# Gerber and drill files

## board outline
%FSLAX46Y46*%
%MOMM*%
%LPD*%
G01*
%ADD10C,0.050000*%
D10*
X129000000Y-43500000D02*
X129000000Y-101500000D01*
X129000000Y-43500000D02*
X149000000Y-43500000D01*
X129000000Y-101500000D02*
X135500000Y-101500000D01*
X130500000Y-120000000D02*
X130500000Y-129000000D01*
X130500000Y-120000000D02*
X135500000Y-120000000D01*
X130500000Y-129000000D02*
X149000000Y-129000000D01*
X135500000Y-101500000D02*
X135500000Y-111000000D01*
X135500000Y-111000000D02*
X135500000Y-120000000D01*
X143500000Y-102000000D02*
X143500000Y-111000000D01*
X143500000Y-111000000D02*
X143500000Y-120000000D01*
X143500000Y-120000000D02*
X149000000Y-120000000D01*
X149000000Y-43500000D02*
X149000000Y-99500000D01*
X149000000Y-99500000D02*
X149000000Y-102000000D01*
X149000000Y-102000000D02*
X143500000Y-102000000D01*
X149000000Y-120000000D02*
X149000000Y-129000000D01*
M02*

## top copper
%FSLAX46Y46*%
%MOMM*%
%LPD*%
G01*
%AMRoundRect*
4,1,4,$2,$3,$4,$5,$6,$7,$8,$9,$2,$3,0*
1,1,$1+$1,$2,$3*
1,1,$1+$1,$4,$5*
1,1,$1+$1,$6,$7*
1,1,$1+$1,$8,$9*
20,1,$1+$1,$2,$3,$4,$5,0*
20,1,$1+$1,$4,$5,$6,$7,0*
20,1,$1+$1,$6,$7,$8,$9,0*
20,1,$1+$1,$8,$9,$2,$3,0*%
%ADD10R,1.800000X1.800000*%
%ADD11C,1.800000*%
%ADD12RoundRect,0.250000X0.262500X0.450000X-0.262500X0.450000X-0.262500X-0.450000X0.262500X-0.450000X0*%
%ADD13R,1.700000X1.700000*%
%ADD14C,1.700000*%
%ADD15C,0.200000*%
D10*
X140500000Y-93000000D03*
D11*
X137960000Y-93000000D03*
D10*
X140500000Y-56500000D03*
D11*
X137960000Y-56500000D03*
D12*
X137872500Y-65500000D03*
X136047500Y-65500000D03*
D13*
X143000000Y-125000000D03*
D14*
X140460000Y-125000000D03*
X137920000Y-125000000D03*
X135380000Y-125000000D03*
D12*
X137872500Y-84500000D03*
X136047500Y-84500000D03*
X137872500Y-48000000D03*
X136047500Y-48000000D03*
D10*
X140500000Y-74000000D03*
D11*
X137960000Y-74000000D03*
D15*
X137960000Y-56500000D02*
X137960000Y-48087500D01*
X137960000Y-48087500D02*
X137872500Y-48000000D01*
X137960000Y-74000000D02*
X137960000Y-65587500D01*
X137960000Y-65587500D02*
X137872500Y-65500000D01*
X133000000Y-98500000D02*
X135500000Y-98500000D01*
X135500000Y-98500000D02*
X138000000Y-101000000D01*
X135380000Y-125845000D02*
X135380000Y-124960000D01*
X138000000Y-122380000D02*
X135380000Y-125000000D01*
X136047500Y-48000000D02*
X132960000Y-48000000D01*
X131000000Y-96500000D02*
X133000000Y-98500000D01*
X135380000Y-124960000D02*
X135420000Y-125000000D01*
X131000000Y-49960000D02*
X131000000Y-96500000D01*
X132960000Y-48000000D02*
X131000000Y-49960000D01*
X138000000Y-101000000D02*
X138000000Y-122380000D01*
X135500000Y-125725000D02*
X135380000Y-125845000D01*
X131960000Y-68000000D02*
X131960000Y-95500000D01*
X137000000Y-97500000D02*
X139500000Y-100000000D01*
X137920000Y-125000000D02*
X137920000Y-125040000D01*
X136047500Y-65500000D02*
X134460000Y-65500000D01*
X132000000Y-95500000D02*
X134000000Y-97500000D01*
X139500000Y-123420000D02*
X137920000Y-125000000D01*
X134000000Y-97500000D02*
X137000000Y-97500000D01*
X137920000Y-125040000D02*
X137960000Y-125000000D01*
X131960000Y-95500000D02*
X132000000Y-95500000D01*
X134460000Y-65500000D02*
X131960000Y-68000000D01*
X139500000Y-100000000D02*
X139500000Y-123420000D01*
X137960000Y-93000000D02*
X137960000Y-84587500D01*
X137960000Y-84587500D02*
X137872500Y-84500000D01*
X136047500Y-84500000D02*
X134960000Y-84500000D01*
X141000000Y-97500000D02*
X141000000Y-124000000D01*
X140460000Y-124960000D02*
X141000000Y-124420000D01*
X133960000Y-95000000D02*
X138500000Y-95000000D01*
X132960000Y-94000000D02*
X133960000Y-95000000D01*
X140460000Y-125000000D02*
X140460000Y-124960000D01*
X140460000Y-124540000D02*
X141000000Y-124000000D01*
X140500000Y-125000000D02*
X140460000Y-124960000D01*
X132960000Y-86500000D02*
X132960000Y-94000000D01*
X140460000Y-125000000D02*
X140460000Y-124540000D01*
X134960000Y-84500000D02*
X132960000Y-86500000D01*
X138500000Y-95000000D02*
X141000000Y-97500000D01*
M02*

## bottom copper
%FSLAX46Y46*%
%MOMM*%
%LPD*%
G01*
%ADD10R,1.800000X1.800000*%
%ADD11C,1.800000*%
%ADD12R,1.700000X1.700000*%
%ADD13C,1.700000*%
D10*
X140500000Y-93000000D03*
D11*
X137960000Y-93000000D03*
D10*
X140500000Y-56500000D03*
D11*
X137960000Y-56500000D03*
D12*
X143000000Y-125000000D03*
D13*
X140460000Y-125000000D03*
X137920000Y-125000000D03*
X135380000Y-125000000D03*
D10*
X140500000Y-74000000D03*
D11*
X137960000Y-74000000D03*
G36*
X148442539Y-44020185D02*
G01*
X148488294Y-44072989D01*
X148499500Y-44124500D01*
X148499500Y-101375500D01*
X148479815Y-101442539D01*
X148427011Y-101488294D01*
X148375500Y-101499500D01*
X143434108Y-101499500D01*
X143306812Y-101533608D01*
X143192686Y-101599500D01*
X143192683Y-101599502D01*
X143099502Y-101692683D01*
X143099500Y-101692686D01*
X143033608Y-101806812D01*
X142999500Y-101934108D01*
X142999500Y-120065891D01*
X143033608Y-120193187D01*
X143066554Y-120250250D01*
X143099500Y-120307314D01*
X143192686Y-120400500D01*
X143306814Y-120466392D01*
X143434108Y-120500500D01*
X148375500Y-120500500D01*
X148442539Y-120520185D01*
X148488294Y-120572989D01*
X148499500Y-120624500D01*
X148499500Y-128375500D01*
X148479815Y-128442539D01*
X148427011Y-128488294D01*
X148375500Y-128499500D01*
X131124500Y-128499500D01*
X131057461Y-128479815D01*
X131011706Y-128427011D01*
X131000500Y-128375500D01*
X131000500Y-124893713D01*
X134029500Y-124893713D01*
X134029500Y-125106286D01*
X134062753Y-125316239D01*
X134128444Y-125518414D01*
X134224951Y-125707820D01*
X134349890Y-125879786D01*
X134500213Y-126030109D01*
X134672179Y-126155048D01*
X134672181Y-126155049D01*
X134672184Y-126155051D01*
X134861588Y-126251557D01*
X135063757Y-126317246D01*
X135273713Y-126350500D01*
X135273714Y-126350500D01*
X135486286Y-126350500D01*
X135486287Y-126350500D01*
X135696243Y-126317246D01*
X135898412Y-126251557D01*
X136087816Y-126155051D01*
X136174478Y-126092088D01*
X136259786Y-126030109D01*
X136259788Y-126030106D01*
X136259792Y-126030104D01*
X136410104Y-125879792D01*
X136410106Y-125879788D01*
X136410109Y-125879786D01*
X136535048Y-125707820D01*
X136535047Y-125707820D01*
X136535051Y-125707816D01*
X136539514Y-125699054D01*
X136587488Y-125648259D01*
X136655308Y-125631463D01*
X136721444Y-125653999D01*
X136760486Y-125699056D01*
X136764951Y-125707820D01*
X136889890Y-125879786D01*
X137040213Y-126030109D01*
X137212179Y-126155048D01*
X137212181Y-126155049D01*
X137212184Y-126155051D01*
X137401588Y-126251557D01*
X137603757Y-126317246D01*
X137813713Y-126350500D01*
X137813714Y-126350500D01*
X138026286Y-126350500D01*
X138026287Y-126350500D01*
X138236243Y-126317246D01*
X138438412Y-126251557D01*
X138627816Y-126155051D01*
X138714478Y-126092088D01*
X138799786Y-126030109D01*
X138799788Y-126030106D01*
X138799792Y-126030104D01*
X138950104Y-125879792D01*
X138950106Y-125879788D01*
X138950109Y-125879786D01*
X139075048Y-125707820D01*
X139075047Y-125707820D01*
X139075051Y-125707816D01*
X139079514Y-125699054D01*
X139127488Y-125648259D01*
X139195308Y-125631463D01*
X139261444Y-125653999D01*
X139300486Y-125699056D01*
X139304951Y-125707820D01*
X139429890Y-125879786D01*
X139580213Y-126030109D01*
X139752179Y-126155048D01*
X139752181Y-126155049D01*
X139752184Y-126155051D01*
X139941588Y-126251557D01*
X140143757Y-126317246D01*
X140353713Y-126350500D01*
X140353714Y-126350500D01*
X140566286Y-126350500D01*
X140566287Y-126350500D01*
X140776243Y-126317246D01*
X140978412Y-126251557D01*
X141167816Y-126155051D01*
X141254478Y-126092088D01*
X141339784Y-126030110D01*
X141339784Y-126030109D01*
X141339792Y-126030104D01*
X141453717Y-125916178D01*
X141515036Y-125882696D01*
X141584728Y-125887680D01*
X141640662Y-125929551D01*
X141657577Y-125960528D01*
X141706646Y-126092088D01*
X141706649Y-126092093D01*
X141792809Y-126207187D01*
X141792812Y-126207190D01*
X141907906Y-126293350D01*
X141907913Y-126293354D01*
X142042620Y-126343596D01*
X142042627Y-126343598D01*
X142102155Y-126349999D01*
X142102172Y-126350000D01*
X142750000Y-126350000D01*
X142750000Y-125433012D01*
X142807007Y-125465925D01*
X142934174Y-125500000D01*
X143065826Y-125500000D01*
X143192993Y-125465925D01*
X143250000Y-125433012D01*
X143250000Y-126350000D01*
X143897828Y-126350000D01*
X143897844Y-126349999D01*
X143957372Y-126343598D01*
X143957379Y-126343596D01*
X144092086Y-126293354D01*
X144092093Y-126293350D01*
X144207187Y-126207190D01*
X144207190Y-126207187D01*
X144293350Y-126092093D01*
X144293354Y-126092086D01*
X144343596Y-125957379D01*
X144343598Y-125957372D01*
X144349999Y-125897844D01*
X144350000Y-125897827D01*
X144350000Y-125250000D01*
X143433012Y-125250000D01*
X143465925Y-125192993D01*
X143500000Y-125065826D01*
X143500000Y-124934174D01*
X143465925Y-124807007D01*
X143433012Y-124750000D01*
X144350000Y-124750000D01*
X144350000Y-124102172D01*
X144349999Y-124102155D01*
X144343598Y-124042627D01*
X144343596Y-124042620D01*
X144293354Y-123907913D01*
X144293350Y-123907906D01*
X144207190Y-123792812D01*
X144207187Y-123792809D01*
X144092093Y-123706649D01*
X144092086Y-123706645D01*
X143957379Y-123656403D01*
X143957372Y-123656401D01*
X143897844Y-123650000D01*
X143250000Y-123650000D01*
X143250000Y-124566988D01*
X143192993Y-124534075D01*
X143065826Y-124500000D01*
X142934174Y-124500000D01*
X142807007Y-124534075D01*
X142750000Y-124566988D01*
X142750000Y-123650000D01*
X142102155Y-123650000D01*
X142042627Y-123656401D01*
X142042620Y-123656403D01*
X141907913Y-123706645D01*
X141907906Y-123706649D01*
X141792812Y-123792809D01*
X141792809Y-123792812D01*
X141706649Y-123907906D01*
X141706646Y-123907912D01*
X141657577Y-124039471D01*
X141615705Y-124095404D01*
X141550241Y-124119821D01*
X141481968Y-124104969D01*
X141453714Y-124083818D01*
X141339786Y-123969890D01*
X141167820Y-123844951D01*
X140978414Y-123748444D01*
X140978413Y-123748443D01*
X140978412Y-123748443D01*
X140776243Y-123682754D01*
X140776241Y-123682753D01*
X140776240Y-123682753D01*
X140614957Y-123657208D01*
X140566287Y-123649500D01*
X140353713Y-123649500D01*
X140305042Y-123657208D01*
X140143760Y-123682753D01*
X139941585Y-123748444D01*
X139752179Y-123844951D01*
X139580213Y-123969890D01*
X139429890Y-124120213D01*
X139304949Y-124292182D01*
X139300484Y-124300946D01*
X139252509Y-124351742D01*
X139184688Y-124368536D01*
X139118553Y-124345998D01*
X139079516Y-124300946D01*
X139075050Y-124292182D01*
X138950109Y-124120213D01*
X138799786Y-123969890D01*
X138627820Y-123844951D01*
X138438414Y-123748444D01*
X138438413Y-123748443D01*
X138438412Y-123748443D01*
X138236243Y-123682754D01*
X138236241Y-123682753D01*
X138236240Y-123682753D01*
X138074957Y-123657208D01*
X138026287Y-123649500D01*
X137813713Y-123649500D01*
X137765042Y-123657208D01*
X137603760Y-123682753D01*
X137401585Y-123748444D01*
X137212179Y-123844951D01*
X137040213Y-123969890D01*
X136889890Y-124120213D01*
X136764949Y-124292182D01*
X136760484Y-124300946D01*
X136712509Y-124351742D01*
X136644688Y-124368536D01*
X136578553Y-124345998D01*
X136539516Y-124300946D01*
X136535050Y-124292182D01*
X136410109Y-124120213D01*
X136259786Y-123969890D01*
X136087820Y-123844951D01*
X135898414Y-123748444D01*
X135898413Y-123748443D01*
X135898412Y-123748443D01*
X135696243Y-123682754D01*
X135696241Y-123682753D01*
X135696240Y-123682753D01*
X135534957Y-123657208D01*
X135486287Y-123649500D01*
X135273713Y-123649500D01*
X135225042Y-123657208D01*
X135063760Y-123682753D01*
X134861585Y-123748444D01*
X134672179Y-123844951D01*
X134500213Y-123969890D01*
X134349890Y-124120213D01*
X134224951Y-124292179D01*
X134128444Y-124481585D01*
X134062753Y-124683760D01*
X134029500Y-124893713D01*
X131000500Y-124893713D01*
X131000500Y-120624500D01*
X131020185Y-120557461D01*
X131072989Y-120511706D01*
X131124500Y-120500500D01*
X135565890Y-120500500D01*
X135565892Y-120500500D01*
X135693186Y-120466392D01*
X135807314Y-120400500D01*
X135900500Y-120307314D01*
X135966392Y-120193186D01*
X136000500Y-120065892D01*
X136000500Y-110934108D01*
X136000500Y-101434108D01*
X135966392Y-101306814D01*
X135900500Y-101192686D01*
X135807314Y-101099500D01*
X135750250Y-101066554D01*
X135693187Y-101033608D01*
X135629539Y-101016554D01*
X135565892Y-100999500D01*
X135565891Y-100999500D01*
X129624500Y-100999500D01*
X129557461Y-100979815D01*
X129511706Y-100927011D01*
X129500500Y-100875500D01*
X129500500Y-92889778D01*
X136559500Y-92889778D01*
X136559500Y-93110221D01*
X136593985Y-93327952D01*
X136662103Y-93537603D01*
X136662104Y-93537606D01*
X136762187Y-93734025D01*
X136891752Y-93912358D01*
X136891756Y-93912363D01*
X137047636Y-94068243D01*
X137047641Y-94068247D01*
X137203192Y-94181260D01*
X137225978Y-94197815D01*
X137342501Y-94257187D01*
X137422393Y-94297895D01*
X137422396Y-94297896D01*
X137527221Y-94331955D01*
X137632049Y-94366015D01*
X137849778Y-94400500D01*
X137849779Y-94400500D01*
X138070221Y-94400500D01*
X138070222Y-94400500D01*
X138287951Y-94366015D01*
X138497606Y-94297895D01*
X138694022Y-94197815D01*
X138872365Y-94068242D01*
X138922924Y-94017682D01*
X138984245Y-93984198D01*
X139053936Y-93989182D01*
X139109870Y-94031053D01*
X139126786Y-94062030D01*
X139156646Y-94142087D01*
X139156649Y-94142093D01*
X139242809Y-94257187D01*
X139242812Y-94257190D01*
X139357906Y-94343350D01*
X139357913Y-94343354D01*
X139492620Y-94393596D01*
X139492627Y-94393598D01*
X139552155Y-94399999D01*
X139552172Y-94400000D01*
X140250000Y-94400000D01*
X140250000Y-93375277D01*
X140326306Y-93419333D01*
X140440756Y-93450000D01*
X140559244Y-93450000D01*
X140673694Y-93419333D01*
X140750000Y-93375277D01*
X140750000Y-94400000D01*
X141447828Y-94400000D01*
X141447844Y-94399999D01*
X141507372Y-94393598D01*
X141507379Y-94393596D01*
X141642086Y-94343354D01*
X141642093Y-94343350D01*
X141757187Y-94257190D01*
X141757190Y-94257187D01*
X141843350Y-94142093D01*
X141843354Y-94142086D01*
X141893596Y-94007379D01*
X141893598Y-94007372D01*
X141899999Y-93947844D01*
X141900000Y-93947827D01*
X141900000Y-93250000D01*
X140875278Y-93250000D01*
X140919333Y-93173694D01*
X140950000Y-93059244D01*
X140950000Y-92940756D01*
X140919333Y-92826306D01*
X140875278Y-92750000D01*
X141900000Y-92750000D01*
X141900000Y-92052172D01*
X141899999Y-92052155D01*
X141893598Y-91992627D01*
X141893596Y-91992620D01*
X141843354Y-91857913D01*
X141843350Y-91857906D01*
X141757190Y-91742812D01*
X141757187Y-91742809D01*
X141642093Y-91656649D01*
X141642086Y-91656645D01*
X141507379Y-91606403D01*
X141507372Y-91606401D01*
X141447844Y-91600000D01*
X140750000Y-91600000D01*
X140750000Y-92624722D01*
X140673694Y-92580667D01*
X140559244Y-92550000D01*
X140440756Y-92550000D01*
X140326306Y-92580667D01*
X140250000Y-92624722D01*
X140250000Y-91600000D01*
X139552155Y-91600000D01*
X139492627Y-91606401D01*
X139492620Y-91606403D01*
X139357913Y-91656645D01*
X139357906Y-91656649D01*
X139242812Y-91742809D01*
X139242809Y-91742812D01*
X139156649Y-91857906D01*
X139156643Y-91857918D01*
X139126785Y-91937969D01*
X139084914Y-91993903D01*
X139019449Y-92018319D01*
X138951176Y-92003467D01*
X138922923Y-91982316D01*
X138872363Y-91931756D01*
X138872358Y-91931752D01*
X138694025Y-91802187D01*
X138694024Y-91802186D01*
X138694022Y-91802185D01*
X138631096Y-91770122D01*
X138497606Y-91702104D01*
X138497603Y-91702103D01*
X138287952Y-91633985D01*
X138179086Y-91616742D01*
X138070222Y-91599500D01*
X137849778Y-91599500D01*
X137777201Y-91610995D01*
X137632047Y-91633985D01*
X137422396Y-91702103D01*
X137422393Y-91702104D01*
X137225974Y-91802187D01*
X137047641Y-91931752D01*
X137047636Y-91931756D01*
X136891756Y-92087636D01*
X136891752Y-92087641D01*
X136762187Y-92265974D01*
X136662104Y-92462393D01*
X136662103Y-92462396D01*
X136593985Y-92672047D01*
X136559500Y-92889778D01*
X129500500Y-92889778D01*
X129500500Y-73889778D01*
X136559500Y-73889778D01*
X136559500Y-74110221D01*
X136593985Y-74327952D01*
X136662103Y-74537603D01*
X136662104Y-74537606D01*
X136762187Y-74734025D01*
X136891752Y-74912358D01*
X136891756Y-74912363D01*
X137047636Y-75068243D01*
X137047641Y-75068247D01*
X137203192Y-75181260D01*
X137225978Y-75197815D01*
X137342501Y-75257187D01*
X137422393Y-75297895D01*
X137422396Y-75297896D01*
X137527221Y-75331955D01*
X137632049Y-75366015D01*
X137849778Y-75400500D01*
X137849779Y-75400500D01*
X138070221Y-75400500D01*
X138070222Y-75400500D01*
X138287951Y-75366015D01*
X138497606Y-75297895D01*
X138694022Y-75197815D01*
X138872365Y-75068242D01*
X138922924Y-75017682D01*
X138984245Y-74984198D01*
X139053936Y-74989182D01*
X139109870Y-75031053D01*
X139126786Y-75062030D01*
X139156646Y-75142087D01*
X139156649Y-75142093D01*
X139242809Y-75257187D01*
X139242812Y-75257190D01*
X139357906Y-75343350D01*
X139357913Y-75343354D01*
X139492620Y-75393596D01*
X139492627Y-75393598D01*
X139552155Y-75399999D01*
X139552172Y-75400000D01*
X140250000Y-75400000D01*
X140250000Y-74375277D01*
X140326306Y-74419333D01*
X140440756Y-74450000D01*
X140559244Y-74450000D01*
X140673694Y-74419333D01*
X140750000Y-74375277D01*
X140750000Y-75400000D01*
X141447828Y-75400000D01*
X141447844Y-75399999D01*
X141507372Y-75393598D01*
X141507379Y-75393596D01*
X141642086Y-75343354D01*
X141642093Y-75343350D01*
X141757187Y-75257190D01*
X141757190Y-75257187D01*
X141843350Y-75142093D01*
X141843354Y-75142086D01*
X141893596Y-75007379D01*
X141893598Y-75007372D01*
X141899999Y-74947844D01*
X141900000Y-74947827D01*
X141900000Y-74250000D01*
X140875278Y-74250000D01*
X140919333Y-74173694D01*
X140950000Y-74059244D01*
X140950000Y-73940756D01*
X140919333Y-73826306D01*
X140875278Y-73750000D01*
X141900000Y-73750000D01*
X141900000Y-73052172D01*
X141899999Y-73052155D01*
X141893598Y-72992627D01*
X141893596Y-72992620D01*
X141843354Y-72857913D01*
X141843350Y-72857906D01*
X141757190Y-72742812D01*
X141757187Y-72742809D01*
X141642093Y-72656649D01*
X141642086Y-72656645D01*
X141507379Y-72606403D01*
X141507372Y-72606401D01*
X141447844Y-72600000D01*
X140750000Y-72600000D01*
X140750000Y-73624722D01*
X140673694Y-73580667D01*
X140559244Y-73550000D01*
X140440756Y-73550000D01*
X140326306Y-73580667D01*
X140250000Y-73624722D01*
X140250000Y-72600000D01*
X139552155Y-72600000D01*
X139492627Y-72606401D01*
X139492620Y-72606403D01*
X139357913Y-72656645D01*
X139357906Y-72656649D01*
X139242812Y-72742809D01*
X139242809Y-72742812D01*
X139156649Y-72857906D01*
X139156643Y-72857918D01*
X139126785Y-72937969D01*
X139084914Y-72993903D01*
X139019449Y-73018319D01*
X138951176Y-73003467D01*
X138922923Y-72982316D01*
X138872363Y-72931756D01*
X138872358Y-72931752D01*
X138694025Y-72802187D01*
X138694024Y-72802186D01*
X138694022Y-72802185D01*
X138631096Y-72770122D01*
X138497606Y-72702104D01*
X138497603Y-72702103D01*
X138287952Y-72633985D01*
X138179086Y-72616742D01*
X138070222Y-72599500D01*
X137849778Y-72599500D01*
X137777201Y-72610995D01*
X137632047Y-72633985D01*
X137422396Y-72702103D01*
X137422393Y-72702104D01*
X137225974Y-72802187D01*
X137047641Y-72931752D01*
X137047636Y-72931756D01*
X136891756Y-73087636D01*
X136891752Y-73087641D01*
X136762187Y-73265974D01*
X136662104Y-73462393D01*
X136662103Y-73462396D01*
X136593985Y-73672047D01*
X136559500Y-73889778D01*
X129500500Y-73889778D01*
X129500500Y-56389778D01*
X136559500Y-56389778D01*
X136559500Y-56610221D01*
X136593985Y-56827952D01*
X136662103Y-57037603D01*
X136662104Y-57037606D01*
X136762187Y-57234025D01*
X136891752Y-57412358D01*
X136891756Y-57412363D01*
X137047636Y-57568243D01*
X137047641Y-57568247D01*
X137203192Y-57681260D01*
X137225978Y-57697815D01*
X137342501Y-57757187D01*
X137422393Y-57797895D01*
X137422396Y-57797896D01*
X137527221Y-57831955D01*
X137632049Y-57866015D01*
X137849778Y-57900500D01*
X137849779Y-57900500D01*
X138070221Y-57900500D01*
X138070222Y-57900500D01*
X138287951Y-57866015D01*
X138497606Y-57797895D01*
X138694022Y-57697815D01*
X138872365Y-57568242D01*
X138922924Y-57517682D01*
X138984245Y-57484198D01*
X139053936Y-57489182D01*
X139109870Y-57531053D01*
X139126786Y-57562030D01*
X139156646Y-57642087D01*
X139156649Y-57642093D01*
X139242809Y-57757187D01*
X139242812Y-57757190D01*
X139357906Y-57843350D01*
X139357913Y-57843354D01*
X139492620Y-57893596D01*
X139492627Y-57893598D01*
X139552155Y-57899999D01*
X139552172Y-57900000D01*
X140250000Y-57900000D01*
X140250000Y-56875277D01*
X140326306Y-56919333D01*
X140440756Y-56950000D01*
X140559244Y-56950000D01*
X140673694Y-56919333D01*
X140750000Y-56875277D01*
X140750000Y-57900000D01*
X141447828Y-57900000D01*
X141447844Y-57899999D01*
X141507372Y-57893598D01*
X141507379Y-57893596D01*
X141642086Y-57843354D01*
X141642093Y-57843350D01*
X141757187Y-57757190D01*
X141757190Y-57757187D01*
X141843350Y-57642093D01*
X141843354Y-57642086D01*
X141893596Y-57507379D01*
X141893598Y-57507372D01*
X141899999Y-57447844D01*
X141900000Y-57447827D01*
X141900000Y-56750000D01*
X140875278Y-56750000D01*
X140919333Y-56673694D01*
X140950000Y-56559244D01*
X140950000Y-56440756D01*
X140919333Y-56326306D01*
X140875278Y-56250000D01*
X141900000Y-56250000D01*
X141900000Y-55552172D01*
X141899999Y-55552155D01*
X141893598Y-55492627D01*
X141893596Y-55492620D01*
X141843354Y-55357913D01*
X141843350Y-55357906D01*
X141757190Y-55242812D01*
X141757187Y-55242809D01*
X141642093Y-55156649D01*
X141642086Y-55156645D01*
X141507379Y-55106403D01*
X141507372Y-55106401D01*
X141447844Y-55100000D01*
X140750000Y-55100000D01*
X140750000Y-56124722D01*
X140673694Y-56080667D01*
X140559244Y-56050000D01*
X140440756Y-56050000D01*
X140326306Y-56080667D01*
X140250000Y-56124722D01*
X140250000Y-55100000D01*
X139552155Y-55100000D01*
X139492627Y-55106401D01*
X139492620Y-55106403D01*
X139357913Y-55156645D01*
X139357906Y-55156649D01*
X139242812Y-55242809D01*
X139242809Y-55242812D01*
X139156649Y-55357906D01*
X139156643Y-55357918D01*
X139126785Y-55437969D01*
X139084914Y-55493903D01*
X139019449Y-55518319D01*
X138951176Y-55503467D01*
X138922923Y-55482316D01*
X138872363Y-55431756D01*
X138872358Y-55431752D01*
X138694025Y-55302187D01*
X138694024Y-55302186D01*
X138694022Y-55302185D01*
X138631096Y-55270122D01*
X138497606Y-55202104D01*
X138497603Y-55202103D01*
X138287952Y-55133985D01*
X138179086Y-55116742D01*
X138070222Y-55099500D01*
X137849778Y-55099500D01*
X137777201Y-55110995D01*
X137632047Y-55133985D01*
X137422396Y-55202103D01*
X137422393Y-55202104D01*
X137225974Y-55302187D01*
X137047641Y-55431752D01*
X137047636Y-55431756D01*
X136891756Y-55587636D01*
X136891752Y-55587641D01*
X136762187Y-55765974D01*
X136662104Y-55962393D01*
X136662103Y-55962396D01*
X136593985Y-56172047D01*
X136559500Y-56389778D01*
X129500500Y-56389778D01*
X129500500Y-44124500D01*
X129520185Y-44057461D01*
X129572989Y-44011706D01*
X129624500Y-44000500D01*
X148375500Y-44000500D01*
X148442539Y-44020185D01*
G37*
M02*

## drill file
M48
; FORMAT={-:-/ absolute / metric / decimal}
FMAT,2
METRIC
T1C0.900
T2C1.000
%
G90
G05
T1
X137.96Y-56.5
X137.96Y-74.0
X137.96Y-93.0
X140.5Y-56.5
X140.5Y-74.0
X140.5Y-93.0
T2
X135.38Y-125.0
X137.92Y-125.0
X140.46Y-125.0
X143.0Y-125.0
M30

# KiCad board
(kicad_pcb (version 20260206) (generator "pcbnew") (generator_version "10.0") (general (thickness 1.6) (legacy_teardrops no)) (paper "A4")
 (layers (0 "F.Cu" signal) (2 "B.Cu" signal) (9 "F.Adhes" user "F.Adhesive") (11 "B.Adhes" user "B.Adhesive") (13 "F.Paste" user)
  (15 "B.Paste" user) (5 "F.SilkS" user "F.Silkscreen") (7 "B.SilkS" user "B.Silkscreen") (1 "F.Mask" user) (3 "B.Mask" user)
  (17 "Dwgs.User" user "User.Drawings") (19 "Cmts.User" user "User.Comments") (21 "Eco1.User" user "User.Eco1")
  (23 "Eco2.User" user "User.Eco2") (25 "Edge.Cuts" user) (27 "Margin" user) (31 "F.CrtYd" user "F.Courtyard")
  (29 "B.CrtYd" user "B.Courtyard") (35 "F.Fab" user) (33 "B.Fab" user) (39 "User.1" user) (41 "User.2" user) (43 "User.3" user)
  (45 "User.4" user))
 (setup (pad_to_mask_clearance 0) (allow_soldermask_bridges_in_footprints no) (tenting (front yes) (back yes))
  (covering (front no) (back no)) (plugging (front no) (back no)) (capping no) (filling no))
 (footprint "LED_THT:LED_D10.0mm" (layer "F.Cu") (at 140.5 93 180)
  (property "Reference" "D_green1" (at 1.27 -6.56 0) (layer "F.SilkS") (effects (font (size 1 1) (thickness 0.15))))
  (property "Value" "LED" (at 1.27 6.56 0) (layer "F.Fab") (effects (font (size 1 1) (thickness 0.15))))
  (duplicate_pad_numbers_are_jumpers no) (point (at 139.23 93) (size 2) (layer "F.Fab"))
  (pad "1" thru_hole rect (at 0 0 180) (size 1.8 1.8) (drill 0.9) (layers "*.Cu" "*.Mask") (remove_unused_layers no) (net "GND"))
  (pad "2" thru_hole circle (at 2.54 0 180) (size 1.8 1.8) (drill 0.9) (layers "*.Cu" "*.Mask") (remove_unused_layers no)
   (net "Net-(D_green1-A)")))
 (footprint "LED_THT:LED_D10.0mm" (layer "F.Cu") (at 140.5 56.5 180)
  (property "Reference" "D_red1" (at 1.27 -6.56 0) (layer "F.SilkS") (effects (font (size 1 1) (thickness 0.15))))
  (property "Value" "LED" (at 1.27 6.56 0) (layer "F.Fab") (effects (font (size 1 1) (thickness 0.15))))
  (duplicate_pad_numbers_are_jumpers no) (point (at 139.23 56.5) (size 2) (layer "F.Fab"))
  (pad "1" thru_hole rect (at 0 0 180) (size 1.8 1.8) (drill 0.9) (layers "*.Cu" "*.Mask") (remove_unused_layers no) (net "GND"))
  (pad "2" thru_hole circle (at 2.54 0 180) (size 1.8 1.8) (drill 0.9) (layers "*.Cu" "*.Mask") (remove_unused_layers no)
   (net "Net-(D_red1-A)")))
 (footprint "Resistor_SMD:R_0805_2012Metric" (layer "F.Cu") (at 136.96 65.5 180)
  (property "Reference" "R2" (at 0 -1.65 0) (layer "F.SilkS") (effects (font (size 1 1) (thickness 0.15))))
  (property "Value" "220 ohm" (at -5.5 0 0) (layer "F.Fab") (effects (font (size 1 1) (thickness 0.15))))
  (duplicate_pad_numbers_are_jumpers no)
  (pad "1" smd roundrect (at -0.9125 0 180) (size 1.025 1.4) (layers "F.Cu" "F.Mask" "F.Paste") (roundrect_rratio 0.243902)
   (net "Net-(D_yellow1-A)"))
  (pad "2" smd roundrect (at 0.9125 0 180) (size 1.025 1.4) (layers "F.Cu" "F.Mask" "F.Paste") (roundrect_rratio 0.243902)
   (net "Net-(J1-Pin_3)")))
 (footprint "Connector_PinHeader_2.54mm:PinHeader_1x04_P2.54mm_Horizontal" (layer "F.Cu") (at 143 125 -90)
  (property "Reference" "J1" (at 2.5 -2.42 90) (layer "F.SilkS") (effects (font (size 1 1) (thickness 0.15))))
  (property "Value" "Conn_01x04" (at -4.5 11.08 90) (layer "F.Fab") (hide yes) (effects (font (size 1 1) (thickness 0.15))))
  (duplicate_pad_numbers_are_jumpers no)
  (pad "1" thru_hole rect (at 0 0 270) (size 1.7 1.7) (drill 1) (layers "*.Cu" "*.Mask") (remove_unused_layers no) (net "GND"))
  (pad "2" thru_hole circle (at 0 2.54 270) (size 1.7 1.7) (drill 1) (layers "*.Cu" "*.Mask") (remove_unused_layers no)
   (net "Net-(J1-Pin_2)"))
  (pad "3" thru_hole circle (at 0 5.08 270) (size 1.7 1.7) (drill 1) (layers "*.Cu" "*.Mask") (remove_unused_layers no)
   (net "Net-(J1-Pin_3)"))
  (pad "4" thru_hole circle (at 0 7.62 270) (size 1.7 1.7) (drill 1) (layers "*.Cu" "*.Mask") (remove_unused_layers no)
   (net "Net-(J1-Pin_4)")))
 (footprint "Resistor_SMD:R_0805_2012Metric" (layer "F.Cu") (at 136.96 84.5 180)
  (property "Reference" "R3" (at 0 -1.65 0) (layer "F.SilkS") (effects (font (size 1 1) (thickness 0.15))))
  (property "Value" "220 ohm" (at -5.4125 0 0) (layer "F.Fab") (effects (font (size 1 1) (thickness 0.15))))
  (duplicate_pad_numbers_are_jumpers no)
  (pad "1" smd roundrect (at -0.9125 0 180) (size 1.025 1.4) (layers "F.Cu" "F.Mask" "F.Paste") (roundrect_rratio 0.243902)
   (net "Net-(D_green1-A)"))
  (pad "2" smd roundrect (at 0.9125 0 180) (size 1.025 1.4) (layers "F.Cu" "F.Mask" "F.Paste") (roundrect_rratio 0.243902)
   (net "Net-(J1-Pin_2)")))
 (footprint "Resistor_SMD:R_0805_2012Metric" (layer "F.Cu") (at 136.96 48 180)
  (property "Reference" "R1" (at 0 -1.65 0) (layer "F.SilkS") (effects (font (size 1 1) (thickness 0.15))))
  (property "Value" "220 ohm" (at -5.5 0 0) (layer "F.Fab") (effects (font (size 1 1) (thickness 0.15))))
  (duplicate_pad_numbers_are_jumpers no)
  (pad "1" smd roundrect (at -0.9125 0 180) (size 1.025 1.4) (layers "F.Cu" "F.Mask" "F.Paste") (roundrect_rratio 0.243902)
   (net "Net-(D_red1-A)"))
  (pad "2" smd roundrect (at 0.9125 0 180) (size 1.025 1.4) (layers "F.Cu" "F.Mask" "F.Paste") (roundrect_rratio 0.243902)
   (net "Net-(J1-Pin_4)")))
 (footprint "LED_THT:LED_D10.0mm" (layer "F.Cu") (at 140.5 74 180)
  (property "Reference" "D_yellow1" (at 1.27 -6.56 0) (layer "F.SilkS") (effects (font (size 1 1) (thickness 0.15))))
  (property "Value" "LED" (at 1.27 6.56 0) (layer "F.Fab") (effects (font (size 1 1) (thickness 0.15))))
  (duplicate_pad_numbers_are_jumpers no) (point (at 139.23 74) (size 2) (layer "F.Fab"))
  (pad "1" thru_hole rect (at 0 0 180) (size 1.8 1.8) (drill 0.9) (layers "*.Cu" "*.Mask") (remove_unused_layers no) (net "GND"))
  (pad "2" thru_hole circle (at 2.54 0 180) (size 1.8 1.8) (drill 0.9) (layers "*.Cu" "*.Mask") (remove_unused_layers no)
   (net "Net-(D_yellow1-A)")))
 (gr_line (start 129 43.5) (end 129 101.5) (stroke (width 0.05) (type default)) (layer "Edge.Cuts"))
 (gr_line (start 129 43.5) (end 149 43.5) (stroke (width 0.05) (type default)) (layer "Edge.Cuts"))
 (gr_line (start 129 101.5) (end 135.5 101.5) (stroke (width 0.05) (type default)) (layer "Edge.Cuts"))
 (gr_line (start 130.5 120) (end 130.5 129) (stroke (width 0.05) (type default)) (layer "Edge.Cuts"))
 (gr_line (start 130.5 120) (end 135.5 120) (stroke (width 0.05) (type default)) (layer "Edge.Cuts"))
 (gr_line (start 130.5 129) (end 149 129) (stroke (width 0.05) (type default)) (layer "Edge.Cuts"))
 (gr_line (start 135.5 101.5) (end 135.5 111) (stroke (width 0.05) (type default)) (layer "Edge.Cuts"))
 (gr_line (start 135.5 111) (end 135.5 120) (stroke (width 0.05) (type default)) (layer "Edge.Cuts"))
 (gr_line (start 143.5 102) (end 143.5 111) (stroke (width 0.05) (type default)) (layer "Edge.Cuts"))
 (gr_line (start 143.5 111) (end 143.5 120) (stroke (width 0.05) (type default)) (layer "Edge.Cuts"))
 (gr_line (start 143.5 120) (end 149 120) (stroke (width 0.05) (type default)) (layer "Edge.Cuts"))
 (gr_line (start 149 43.5) (end 149 99.5) (stroke (width 0.05) (type default)) (layer "Edge.Cuts"))
 (gr_line (start 149 99.5) (end 149 102) (stroke (width 0.05) (type default)) (layer "Edge.Cuts"))
 (gr_line (start 149 102) (end 143.5 102) (stroke (width 0.05) (type default)) (layer "Edge.Cuts"))
 (gr_line (start 149 120) (end 149 129) (stroke (width 0.05) (type default)) (layer "Edge.Cuts"))
 (segment (start 137.96 56.5) (end 137.96 48.0875) (width 0.2) (layer "F.Cu") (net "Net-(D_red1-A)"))
 (segment (start 137.96 48.0875) (end 137.8725 48) (width 0.2) (layer "F.Cu") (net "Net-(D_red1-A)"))
 (segment (start 137.96 74) (end 137.96 65.5875) (width 0.2) (layer "F.Cu") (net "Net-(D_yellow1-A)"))
 (segment (start 137.96 65.5875) (end 137.8725 65.5) (width 0.2) (layer "F.Cu") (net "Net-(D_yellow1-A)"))
 (segment (start 133 98.5) (end 135.5 98.5) (width 0.2) (layer "F.Cu") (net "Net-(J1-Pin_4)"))
 (segment (start 135.5 98.5) (end 138 101) (width 0.2) (layer "F.Cu") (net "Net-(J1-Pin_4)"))
 (segment (start 135.38 125.845) (end 135.38 124.96) (width 0.2) (layer "F.Cu") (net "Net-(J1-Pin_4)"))
 (segment (start 138 122.38) (end 135.38 125) (width 0.2) (layer "F.Cu") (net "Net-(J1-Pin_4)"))
 (segment (start 136.0475 48) (end 132.96 48) (width 0.2) (layer "F.Cu") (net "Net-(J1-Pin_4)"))
 (segment (start 131 96.5) (end 133 98.5) (width 0.2) (layer "F.Cu") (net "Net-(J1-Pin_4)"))
 (segment (start 135.38 124.96) (end 135.42 125) (width 0.2) (layer "F.Cu") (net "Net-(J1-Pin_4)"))
 (segment (start 131 49.96) (end 131 96.5) (width 0.2) (layer "F.Cu") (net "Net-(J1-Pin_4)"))
 (segment (start 132.96 48) (end 131 49.96) (width 0.2) (layer "F.Cu") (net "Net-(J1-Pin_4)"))
 (segment (start 138 101) (end 138 122.38) (width 0.2) (layer "F.Cu") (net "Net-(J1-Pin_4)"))
 (segment (start 135.5 125.725) (end 135.38 125.845) (width 0.2) (layer "F.Cu") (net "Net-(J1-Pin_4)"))
 (segment (start 131.96 68) (end 131.96 95.5) (width 0.2) (layer "F.Cu") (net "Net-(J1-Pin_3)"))
 (segment (start 137 97.5) (end 139.5 100) (width 0.2) (layer "F.Cu") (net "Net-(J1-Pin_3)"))
 (segment (start 137.92 125) (end 137.92 125.04) (width 0.2) (layer "F.Cu") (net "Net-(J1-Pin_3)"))
 (segment (start 136.0475 65.5) (end 134.46 65.5) (width 0.2) (layer "F.Cu") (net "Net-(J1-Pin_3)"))
 (segment (start 132 95.5) (end 134 97.5) (width 0.2) (layer "F.Cu") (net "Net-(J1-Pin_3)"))
 (segment (start 139.5 123.42) (end 137.92 125) (width 0.2) (layer "F.Cu") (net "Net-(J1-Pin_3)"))
 (segment (start 134 97.5) (end 137 97.5) (width 0.2) (layer "F.Cu") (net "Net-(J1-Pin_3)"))
 (segment (start 137.92 125.04) (end 137.96 125) (width 0.2) (layer "F.Cu") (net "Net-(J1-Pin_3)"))
 (segment (start 131.96 95.5) (end 132 95.5) (width 0.2) (layer "F.Cu") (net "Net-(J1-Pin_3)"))
 (segment (start 134.46 65.5) (end 131.96 68) (width 0.2) (layer "F.Cu") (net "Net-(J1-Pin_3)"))
 (segment (start 139.5 100) (end 139.5 123.42) (width 0.2) (layer "F.Cu") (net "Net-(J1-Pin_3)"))
 (segment (start 137.96 93) (end 137.96 84.5875) (width 0.2) (layer "F.Cu") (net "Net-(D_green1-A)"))
 (segment (start 137.96 84.5875) (end 137.8725 84.5) (width 0.2) (layer "F.Cu") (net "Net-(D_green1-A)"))
 (segment (start 136.0475 84.5) (end 134.96 84.5) (width 0.2) (layer "F.Cu") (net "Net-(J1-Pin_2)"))
 (segment (start 141 97.5) (end 141 124) (width 0.2) (layer "F.Cu") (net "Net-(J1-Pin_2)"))
 (segment (start 140.46 124.96) (end 141 124.42) (width 0.2) (layer "F.Cu") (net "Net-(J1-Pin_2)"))
 (segment (start 133.96 95) (end 138.5 95) (width 0.2) (layer "F.Cu") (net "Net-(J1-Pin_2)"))
 (segment (start 132.96 94) (end 133.96 95) (width 0.2) (layer "F.Cu") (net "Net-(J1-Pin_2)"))
 (segment (start 140.46 125) (end 140.46 124.96) (width 0.2) (layer "F.Cu") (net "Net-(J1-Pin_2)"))
 (segment (start 140.46 124.54) (end 141 124) (width 0.2) (layer "F.Cu") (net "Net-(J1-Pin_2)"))
 (segment (start 140.5 125) (end 140.46 124.96) (width 0.2) (layer "F.Cu") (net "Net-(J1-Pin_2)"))
 (segment (start 132.96 86.5) (end 132.96 94) (width 0.2) (layer "F.Cu") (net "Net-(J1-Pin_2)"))
 (segment (start 140.46 125) (end 140.46 124.54) (width 0.2) (layer "F.Cu") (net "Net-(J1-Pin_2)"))
 (segment (start 134.96 84.5) (end 132.96 86.5) (width 0.2) (layer "F.Cu") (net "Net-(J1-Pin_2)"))
 (segment (start 138.5 95) (end 141 97.5) (width 0.2) (layer "F.Cu") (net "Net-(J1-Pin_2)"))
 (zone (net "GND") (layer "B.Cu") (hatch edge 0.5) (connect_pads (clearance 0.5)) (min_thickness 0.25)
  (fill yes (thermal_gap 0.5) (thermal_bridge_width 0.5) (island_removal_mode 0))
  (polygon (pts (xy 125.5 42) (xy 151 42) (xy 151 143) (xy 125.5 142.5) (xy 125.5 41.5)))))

